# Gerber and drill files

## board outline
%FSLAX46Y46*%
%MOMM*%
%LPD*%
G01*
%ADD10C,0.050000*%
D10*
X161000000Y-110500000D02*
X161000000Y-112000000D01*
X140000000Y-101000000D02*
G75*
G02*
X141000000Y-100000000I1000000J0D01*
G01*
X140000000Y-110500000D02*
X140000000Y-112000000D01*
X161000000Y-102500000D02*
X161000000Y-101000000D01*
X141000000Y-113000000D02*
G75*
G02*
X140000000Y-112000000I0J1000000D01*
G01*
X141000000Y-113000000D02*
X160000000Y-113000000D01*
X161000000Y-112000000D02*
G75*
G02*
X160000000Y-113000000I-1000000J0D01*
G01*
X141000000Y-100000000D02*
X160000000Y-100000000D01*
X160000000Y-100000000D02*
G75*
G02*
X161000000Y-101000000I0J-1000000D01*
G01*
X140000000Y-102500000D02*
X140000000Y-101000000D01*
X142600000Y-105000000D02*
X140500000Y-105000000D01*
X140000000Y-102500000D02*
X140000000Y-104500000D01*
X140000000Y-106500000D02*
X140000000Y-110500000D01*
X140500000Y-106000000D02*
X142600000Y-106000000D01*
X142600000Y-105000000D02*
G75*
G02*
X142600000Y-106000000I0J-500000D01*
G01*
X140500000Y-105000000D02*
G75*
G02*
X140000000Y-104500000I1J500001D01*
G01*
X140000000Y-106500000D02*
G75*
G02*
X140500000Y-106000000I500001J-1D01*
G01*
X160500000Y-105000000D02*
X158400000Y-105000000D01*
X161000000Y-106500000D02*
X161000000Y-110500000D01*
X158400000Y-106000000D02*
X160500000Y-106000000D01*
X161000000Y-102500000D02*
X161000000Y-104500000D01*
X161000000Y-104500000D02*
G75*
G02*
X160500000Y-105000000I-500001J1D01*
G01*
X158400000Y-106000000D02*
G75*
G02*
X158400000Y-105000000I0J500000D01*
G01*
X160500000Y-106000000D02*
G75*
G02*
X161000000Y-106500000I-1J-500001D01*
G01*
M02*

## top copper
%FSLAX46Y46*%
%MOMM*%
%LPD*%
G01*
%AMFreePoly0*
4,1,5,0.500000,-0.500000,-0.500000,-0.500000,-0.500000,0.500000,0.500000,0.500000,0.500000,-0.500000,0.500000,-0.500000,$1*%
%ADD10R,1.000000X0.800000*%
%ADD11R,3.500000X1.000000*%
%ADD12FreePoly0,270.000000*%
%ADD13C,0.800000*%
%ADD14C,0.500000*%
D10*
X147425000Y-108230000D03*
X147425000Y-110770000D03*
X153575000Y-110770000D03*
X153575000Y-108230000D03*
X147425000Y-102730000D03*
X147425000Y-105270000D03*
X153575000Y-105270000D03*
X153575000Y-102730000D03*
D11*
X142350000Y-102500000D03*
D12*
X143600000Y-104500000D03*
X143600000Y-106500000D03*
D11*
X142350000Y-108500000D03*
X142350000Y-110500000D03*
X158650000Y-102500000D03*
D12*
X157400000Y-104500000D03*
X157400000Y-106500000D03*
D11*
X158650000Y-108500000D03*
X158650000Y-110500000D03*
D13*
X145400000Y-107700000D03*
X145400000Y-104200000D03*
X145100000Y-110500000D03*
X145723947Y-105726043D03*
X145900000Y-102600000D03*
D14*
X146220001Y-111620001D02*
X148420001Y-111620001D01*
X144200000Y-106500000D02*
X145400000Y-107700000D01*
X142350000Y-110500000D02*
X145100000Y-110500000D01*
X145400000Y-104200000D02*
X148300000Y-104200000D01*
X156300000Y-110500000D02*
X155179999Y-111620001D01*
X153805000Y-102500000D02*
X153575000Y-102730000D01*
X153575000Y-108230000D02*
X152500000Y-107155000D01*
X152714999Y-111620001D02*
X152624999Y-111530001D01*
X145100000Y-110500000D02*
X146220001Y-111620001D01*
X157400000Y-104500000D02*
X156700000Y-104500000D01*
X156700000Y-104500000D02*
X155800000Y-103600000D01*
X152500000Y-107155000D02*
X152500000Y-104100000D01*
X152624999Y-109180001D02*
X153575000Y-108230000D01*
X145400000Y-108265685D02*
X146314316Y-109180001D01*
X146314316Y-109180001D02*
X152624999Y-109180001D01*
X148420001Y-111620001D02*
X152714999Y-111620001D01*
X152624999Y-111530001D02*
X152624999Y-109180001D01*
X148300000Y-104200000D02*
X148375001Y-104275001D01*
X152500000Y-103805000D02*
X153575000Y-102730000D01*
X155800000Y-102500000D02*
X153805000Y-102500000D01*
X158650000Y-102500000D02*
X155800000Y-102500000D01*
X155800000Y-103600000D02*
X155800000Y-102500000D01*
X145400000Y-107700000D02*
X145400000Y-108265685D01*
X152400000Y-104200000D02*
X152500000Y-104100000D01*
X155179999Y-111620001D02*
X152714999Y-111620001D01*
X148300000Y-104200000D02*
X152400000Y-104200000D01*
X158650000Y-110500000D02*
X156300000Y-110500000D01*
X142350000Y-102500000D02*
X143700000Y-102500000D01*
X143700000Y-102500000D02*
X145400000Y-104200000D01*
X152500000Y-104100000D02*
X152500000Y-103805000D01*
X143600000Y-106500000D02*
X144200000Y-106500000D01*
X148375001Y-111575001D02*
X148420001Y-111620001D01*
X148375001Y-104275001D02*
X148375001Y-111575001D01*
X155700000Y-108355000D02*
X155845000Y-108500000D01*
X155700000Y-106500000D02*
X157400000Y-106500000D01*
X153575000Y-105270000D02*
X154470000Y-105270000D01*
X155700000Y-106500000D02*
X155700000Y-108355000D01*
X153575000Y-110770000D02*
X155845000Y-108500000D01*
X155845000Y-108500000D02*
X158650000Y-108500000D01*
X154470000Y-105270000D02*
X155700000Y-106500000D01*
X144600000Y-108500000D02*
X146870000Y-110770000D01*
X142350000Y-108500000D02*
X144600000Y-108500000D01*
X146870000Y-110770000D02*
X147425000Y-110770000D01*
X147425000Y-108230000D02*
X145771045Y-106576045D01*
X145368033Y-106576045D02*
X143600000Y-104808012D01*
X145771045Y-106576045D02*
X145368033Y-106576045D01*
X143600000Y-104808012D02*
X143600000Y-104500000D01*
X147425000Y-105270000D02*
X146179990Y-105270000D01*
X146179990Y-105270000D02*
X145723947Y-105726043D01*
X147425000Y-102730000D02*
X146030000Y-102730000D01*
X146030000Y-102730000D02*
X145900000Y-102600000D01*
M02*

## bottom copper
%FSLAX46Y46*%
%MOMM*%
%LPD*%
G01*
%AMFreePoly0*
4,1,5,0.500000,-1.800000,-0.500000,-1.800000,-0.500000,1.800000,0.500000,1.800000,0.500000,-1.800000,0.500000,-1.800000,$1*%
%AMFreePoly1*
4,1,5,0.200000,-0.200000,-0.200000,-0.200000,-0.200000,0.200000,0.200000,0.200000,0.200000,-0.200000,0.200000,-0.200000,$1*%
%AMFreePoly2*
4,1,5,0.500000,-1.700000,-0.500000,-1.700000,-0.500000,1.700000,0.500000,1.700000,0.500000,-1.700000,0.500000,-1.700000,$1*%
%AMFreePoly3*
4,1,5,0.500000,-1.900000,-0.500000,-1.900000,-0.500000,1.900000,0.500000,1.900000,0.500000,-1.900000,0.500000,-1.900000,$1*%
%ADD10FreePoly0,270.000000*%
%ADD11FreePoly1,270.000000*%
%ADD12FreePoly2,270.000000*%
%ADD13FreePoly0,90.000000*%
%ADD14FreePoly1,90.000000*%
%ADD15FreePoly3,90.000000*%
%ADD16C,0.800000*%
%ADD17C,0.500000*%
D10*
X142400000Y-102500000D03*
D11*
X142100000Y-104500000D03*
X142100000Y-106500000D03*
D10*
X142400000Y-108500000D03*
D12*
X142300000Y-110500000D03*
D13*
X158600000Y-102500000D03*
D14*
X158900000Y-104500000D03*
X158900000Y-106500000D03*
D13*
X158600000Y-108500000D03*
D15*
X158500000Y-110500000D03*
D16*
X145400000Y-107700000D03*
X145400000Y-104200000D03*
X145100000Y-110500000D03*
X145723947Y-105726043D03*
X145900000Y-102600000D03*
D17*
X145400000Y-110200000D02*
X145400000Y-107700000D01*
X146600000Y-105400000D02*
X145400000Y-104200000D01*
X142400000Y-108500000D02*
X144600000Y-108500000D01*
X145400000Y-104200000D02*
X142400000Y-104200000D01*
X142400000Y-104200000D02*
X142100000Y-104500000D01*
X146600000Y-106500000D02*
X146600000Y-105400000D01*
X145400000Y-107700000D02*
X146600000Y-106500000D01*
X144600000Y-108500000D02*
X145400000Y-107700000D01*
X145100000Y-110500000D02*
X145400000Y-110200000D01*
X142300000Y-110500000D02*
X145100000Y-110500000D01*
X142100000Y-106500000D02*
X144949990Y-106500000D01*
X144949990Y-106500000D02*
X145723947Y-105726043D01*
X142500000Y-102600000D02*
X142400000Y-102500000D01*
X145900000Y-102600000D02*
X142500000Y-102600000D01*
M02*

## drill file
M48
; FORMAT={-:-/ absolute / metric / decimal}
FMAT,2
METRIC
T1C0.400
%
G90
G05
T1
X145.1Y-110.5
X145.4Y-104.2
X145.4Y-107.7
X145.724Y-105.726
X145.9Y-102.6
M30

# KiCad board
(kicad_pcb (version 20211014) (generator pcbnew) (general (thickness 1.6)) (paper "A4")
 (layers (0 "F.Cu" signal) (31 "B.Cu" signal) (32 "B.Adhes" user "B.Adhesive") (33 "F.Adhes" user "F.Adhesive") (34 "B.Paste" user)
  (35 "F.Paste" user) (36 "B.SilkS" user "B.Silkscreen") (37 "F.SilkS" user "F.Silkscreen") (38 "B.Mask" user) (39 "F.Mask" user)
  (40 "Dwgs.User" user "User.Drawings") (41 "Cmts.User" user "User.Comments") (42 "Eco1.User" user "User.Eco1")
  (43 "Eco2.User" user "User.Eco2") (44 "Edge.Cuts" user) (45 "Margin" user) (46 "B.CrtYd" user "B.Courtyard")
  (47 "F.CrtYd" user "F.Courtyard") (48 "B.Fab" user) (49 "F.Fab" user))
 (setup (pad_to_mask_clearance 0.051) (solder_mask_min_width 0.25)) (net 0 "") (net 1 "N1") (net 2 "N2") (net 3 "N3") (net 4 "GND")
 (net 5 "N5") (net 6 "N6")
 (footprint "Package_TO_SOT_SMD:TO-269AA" (layer "F.Cu") (at 150.5 109.5)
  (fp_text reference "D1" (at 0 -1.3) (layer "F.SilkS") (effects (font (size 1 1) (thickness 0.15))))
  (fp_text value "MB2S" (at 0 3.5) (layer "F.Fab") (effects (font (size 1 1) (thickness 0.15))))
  (pad "1" smd rect locked (at -3.075 -1.27) (size 1 0.8) (layers "F.Cu" "F.Paste" "F.Mask") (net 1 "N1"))
  (pad "2" smd rect locked (at -3.075 1.27) (size 1 0.8) (layers "F.Cu" "F.Paste" "F.Mask") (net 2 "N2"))
  (pad "3" smd rect locked (at 3.075 1.27) (size 1 0.8) (layers "F.Cu" "F.Paste" "F.Mask") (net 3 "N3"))
  (pad "4" smd rect locked (at 3.075 -1.27) (size 1 0.8) (layers "F.Cu" "F.Paste" "F.Mask") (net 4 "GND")))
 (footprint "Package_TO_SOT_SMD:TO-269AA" (layer "F.Cu") (at 150.5 104)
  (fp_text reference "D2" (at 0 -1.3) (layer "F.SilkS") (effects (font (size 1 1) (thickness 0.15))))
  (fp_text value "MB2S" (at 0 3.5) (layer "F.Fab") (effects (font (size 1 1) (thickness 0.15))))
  (pad "1" smd rect locked (at -3.075 -1.27) (size 1 0.8) (layers "F.Cu" "F.Paste" "F.Mask") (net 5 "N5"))
  (pad "2" smd rect locked (at -3.075 1.27) (size 1 0.8) (layers "F.Cu" "F.Paste" "F.Mask") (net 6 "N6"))
  (pad "3" smd rect locked (at 3.075 1.27) (size 1 0.8) (layers "F.Cu" "F.Paste" "F.Mask") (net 3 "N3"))
  (pad "4" smd rect locked (at 3.075 -1.27) (size 1 0.8) (layers "F.Cu" "F.Paste" "F.Mask") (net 4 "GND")))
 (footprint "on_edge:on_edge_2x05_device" (layer "F.Cu") (at 140 106.5 -90)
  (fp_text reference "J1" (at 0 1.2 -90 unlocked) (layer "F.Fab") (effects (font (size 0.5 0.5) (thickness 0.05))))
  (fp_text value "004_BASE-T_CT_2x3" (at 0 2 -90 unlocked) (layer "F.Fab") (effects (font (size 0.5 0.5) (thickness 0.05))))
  (fp_line (start -1.5 -2.6) (end -1.5 -0.5) (layer "Edge.Cuts") (width 0.05))
  (fp_line (start -4 0) (end -2 0) (layer "Edge.Cuts") (width 0.05))
  (fp_line (start 0 0) (end 4 0) (layer "Edge.Cuts") (width 0.05))
  (fp_line (start -0.5 -0.5) (end -0.5 -2.6) (layer "Edge.Cuts") (width 0.05))
  (fp_arc (start -1.5 -2.6) (mid -1 -3.1) (end -0.5 -2.6) (layer "Edge.Cuts") (width 0.05))
  (fp_arc (start -1.5 -0.5) (mid -1.646447 -0.146447) (end -2 0) (layer "Edge.Cuts") (width 0.05))
  (fp_arc (start 0 0) (mid -0.353553 -0.146447) (end -0.5 -0.5) (layer "Edge.Cuts") (width 0.05))
  (pad "1" smd rect locked (at -4 -2.35 90) (size 1 3.5) (layers "F.Cu" "F.Mask") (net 4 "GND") (zone_connect 0))
  (pad "2" smd custom locked (at -2 -3.6 270) (size 1 1) (layers "F.Cu" "F.Mask") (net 1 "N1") (zone_connect 0)
   (options (clearance outline) (anchor rect)) (primitives))
  (pad "3" smd custom locked (at 0 -3.6 270) (size 1 1) (layers "F.Cu" "F.Mask") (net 4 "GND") (zone_connect 0)
   (options (clearance outline) (anchor rect)) (primitives))
  (pad "4" smd rect locked (at 2 -2.35 90) (size 1 3.5) (layers "F.Cu" "F.Mask") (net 2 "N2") (zone_connect 0))
  (pad "5" smd rect locked (at 4 -2.35 90) (size 1 3.5) (layers "F.Cu" "F.Mask") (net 4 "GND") (zone_connect 0))
  (pad "6" smd custom locked (at -4 -2.4 270) (size 1 3.6) (layers "B.Cu" "B.Mask") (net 5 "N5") (zone_connect 0)
   (options (clearance outline) (anchor rect)) (primitives))
  (pad "7" smd custom locked (at -2 -2.1 270) (size 0.4 0.4) (layers "B.Cu" "B.Mask") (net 4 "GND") (zone_connect 0)
   (options (clearance outline) (anchor rect)) (primitives))
  (pad "8" smd custom locked (at 0 -2.1 270) (size 0.4 0.4) (layers "B.Cu" "B.Mask") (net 6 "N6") (zone_connect 0)
   (options (clearance outline) (anchor rect)) (primitives))
  (pad "9" smd custom locked (at 2 -2.4 270) (size 1 3.6) (layers "B.Cu" "B.Mask") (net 4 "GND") (zone_connect 0)
   (options (clearance outline) (anchor rect)) (primitives))
  (pad "10" smd custom locked (at 4 -2.3 270) (size 1 3.4) (layers "B.Cu" "B.Mask") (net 4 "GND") (zone_connect 0)
   (options (clearance outline) (anchor rect)) (primitives)))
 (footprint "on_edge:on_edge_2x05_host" (layer "F.Cu") (at 161 106.5 -90)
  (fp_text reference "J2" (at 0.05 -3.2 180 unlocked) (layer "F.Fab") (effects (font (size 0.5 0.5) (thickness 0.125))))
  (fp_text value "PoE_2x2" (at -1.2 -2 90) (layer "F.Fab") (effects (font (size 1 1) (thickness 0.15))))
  (fp_line (start -1.5 0.5) (end -1.5 2.6) (layer "Edge.Cuts") (width 0.05))
  (fp_line (start 0 0) (end 4 0) (layer "Edge.Cuts") (width 0.05))
  (fp_line (start -0.5 2.6) (end -0.5 0.5) (layer "Edge.Cuts") (width 0.05))
  (fp_line (start -4 0) (end -2 0) (layer "Edge.Cuts") (width 0.05))
  (fp_arc (start -2 0) (mid -1.646447 0.146447) (end -1.5 0.5) (layer "Edge.Cuts") (width 0.05))
  (fp_arc (start -0.5 2.6) (mid -1 3.1) (end -1.5 2.6) (layer "Edge.Cuts") (width 0.05))
  (fp_arc (start -0.5 0.5) (mid -0.353553 0.146447) (end 0 0) (layer "Edge.Cuts") (width 0.05))
  (pad "1" smd rect locked (at -4 2.35 270) (size 1 3.5) (layers "F.Cu" "F.Mask") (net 4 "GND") (zone_connect 0))
  (pad "2" smd custom locked (at -2 3.6 270) (size 1 1) (layers "F.Cu" "F.Mask") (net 4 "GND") (zone_connect 0)
   (options (clearance outline) (anchor rect)) (primitives))
  (pad "3" smd custom locked (at 0 3.6 270) (size 1 1) (layers "F.Cu" "F.Mask") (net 3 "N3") (zone_connect 0)
   (options (clearance outline) (anchor rect)) (primitives))
  (pad "4" smd rect locked (at 2 2.35 270) (size 1 3.5) (layers "F.Cu" "F.Mask") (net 3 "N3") (zone_connect 0))
  (pad "5" smd rect locked (at 4 2.35 270) (size 1 3.5) (layers "F.Cu" "F.Mask") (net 4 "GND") (zone_connect 0))
  (pad "6" smd custom locked (at -4 2.4 90) (size 1 3.6) (layers "B.Cu" "B.Mask") (zone_connect 0)
   (options (clearance outline) (anchor rect)) (primitives))
  (pad "7" smd custom locked (at -2 2.1 90) (size 0.4 0.4) (layers "B.Cu" "B.Mask") (zone_connect 0)
   (options (clearance outline) (anchor rect)) (primitives))
  (pad "8" smd custom locked (at 0 2.1 90) (size 0.4 0.4) (layers "B.Cu" "B.Mask") (zone_connect 0)
   (options (clearance outline) (anchor rect)) (primitives))
  (pad "9" smd custom locked (at 2 2.4 90) (size 1 3.6) (layers "B.Cu" "B.Mask") (zone_connect 0)
   (options (clearance outline) (anchor rect)) (primitives))
  (pad "10" smd custom locked (at 4 2.5 90) (size 1 3.8) (layers "B.Cu" "B.Mask") (zone_connect 0)
   (options (clearance outline) (anchor rect)) (primitives)))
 (gr_line (start 161 110.5) (end 161 112) (layer "Edge.Cuts") (width 0.05))
 (gr_arc (start 140 101) (mid 140.292893 100.292893) (end 141 100) (layer "Edge.Cuts") (width 0.05))
 (gr_line (start 140 110.5) (end 140 112) (layer "Edge.Cuts") (width 0.05))
 (gr_line (start 161 102.5) (end 161 101) (layer "Edge.Cuts") (width 0.05))
 (gr_arc (start 141 113) (mid 140.292893 112.707107) (end 140 112) (layer "Edge.Cuts") (width 0.05))
 (gr_line (start 141 113) (end 160 113) (layer "Edge.Cuts") (width 0.05))
 (gr_arc (start 161 112) (mid 160.707107 112.707107) (end 160 113) (layer "Edge.Cuts") (width 0.05))
 (gr_line (start 141 100) (end 160 100) (layer "Edge.Cuts") (width 0.05))
 (gr_arc (start 160 100) (mid 160.707107 100.292893) (end 161 101) (layer "Edge.Cuts") (width 0.05))
 (gr_line (start 140 102.5) (end 140 101) (layer "Edge.Cuts") (width 0.05))
 (segment (start 146.220001 111.620001) (end 148.420001 111.620001) (width 0.5) (layer "F.Cu") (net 4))
 (segment (start 144.2 106.5) (end 145.4 107.7) (width 0.5) (layer "F.Cu") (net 4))
 (segment (start 142.35 110.5) (end 145.1 110.5) (width 0.5) (layer "F.Cu") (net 4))
 (segment (start 145.4 104.2) (end 148.3 104.2) (width 0.5) (layer "F.Cu") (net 4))
 (segment (start 156.3 110.5) (end 155.179999 111.620001) (width 0.5) (layer "F.Cu") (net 4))
 (segment (start 153.805 102.5) (end 153.575 102.73) (width 0.5) (layer "F.Cu") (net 4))
 (segment (start 153.575 108.23) (end 152.5 107.155) (width 0.5) (layer "F.Cu") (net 4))
 (segment (start 152.714999 111.620001) (end 152.624999 111.530001) (width 0.5) (layer "F.Cu") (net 4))
 (segment (start 145.1 110.5) (end 146.220001 111.620001) (width 0.5) (layer "F.Cu") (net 4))
 (segment (start 157.4 104.5) (end 156.7 104.5) (width 0.5) (layer "F.Cu") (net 4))
 (segment (start 156.7 104.5) (end 155.8 103.6) (width 0.5) (layer "F.Cu") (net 4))
 (segment (start 152.5 107.155) (end 152.5 104.1) (width 0.5) (layer "F.Cu") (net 4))
 (segment (start 152.624999 109.180001) (end 153.575 108.23) (width 0.5) (layer "F.Cu") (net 4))
 (segment (start 145.4 108.265685) (end 146.314316 109.180001) (width 0.5) (layer "F.Cu") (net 4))
 (segment (start 146.314316 109.180001) (end 152.624999 109.180001) (width 0.5) (layer "F.Cu") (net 4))
 (segment (start 148.420001 111.620001) (end 152.714999 111.620001) (width 0.5) (layer "F.Cu") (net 4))
 (segment (start 152.624999 111.530001) (end 152.624999 109.180001) (width 0.5) (layer "F.Cu") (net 4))
 (segment (start 148.3 104.2) (end 148.375001 104.275001) (width 0.5) (layer "F.Cu") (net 4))
 (segment (start 152.5 103.805) (end 153.575 102.73) (width 0.5) (layer "F.Cu") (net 4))
 (segment (start 155.8 102.5) (end 153.805 102.5) (width 0.5) (layer "F.Cu") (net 4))
 (segment (start 158.65 102.5) (end 155.8 102.5) (width 0.5) (layer "F.Cu") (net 4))
 (segment (start 155.8 103.6) (end 155.8 102.5) (width 0.5) (layer "F.Cu") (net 4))
 (segment (start 145.4 107.7) (end 145.4 108.265685) (width 0.5) (layer "F.Cu") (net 4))
 (segment (start 152.4 104.2) (end 152.5 104.1) (width 0.5) (layer "F.Cu") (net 4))
 (segment (start 155.179999 111.620001) (end 152.714999 111.620001) (width 0.5) (layer "F.Cu") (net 4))
 (segment (start 148.3 104.2) (end 152.4 104.2) (width 0.5) (layer "F.Cu") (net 4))
 (segment (start 158.65 110.5) (end 156.3 110.5) (width 0.5) (layer "F.Cu") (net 4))
 (segment (start 142.35 102.5) (end 143.7 102.5) (width 0.5) (layer "F.Cu") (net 4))
 (segment (start 143.7 102.5) (end 145.4 104.2) (width 0.5) (layer "F.Cu") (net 4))
 (segment (start 152.5 104.1) (end 152.5 103.805) (width 0.5) (layer "F.Cu") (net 4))
 (segment (start 143.6 106.5) (end 144.2 106.5) (width 0.5) (layer "F.Cu") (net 4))
 (segment (start 148.375001 111.575001) (end 148.420001 111.620001) (width 0.5) (layer "F.Cu") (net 4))
 (segment (start 148.375001 104.275001) (end 148.375001 111.575001) (width 0.5) (layer "F.Cu") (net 4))
 (via (at 145.4 107.7) (size 0.8) (drill 0.4) (layers "F.Cu" "B.Cu") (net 4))
 (via (at 145.4 104.2) (size 0.8) (drill 0.4) (layers "F.Cu" "B.Cu") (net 4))
 (via (at 145.1 110.5) (size 0.8) (drill 0.4) (layers "F.Cu" "B.Cu") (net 4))
 (segment (start 145.4 110.2) (end 145.4 107.7) (width 0.5) (layer "B.Cu") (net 4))
 (segment (start 146.6 105.4) (end 145.4 104.2) (width 0.5) (layer "B.Cu") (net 4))
 (segment (start 142.4 108.5) (end 144.6 108.5) (width 0.5) (layer "B.Cu") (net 4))
 (segment (start 145.4 104.2) (end 142.4 104.2) (width 0.5) (layer "B.Cu") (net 4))
 (segment (start 142.4 104.2) (end 142.1 104.5) (width 0.5) (layer "B.Cu") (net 4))
 (segment (start 146.6 106.5) (end 146.6 105.4) (width 0.5) (layer "B.Cu") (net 4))
 (segment (start 145.4 107.7) (end 146.6 106.5) (width 0.5) (layer "B.Cu") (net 4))
 (segment (start 144.6 108.5) (end 145.4 107.7) (width 0.5) (layer "B.Cu") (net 4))
 (segment (start 145.1 110.5) (end 145.4 110.2) (width 0.5) (layer "B.Cu") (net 4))
 (segment (start 142.3 110.5) (end 145.1 110.5) (width 0.5) (layer "B.Cu") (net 4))
 (segment (start 155.7 108.355) (end 155.845 108.5) (width 0.5) (layer "F.Cu") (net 3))
 (segment (start 155.7 106.5) (end 157.4 106.5) (width 0.5) (layer "F.Cu") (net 3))
 (segment (start 153.575 105.27) (end 154.47 105.27) (width 0.5) (layer "F.Cu") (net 3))
 (segment (start 155.7 106.5) (end 155.7 108.355) (width 0.5) (layer "F.Cu") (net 3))
 (segment (start 153.575 110.77) (end 155.845 108.5) (width 0.5) (layer "F.Cu") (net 3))
 (segment (start 155.845 108.5) (end 158.65 108.5) (width 0.5) (layer "F.Cu") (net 3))
 (segment (start 154.47 105.27) (end 155.7 106.5) (width 0.5) (layer "F.Cu") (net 3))
 (segment (start 144.6 108.5) (end 146.87 110.77) (width 0.5) (layer "F.Cu") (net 2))
 (segment (start 142.35 108.5) (end 144.6 108.5) (width 0.5) (layer "F.Cu") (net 2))
 (segment (start 146.87 110.77) (end 147.425 110.77) (width 0.5) (layer "F.Cu") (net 2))
 (segment (start 147.425 108.23) (end 145.771045 106.576045) (width 0.5) (layer "F.Cu") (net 1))
 (segment (start 145.368033 106.576045) (end 143.6 104.808012) (width 0.5) (layer "F.Cu") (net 1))
 (segment (start 145.771045 106.576045) (end 145.368033 106.576045) (width 0.5) (layer "F.Cu") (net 1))
 (segment (start 143.6 104.808012) (end 143.6 104.5) (width 0.5) (layer "F.Cu") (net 1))
 (segment (start 147.425 105.27) (end 146.17999 105.27) (width 0.5) (layer "F.Cu") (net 6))
 (segment (start 146.17999 105.27) (end 145.723947 105.726043) (width 0.5) (layer "F.Cu") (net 6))
 (via (at 145.723947 105.726043) (size 0.8) (drill 0.4) (layers "F.Cu" "B.Cu") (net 6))
 (segment (start 142.1 106.5) (end 144.94999 106.5) (width 0.5) (layer "B.Cu") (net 6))
 (segment (start 144.94999 106.5) (end 145.723947 105.726043) (width 0.5) (layer "B.Cu") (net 6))
 (segment (start 147.425 102.73) (end 146.03 102.73) (width 0.5) (layer "F.Cu") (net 5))
 (segment (start 146.03 102.73) (end 145.9 102.6) (width 0.5) (layer "F.Cu") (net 5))
 (via (at 145.9 102.6) (size 0.8) (drill 0.4) (layers "F.Cu" "B.Cu") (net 5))
 (segment (start 142.5 102.6) (end 142.4 102.5) (width 0.5) (layer "B.Cu") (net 5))
 (segment (start 145.9 102.6) (end 142.5 102.6) (width 0.5) (layer "B.Cu") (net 5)))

